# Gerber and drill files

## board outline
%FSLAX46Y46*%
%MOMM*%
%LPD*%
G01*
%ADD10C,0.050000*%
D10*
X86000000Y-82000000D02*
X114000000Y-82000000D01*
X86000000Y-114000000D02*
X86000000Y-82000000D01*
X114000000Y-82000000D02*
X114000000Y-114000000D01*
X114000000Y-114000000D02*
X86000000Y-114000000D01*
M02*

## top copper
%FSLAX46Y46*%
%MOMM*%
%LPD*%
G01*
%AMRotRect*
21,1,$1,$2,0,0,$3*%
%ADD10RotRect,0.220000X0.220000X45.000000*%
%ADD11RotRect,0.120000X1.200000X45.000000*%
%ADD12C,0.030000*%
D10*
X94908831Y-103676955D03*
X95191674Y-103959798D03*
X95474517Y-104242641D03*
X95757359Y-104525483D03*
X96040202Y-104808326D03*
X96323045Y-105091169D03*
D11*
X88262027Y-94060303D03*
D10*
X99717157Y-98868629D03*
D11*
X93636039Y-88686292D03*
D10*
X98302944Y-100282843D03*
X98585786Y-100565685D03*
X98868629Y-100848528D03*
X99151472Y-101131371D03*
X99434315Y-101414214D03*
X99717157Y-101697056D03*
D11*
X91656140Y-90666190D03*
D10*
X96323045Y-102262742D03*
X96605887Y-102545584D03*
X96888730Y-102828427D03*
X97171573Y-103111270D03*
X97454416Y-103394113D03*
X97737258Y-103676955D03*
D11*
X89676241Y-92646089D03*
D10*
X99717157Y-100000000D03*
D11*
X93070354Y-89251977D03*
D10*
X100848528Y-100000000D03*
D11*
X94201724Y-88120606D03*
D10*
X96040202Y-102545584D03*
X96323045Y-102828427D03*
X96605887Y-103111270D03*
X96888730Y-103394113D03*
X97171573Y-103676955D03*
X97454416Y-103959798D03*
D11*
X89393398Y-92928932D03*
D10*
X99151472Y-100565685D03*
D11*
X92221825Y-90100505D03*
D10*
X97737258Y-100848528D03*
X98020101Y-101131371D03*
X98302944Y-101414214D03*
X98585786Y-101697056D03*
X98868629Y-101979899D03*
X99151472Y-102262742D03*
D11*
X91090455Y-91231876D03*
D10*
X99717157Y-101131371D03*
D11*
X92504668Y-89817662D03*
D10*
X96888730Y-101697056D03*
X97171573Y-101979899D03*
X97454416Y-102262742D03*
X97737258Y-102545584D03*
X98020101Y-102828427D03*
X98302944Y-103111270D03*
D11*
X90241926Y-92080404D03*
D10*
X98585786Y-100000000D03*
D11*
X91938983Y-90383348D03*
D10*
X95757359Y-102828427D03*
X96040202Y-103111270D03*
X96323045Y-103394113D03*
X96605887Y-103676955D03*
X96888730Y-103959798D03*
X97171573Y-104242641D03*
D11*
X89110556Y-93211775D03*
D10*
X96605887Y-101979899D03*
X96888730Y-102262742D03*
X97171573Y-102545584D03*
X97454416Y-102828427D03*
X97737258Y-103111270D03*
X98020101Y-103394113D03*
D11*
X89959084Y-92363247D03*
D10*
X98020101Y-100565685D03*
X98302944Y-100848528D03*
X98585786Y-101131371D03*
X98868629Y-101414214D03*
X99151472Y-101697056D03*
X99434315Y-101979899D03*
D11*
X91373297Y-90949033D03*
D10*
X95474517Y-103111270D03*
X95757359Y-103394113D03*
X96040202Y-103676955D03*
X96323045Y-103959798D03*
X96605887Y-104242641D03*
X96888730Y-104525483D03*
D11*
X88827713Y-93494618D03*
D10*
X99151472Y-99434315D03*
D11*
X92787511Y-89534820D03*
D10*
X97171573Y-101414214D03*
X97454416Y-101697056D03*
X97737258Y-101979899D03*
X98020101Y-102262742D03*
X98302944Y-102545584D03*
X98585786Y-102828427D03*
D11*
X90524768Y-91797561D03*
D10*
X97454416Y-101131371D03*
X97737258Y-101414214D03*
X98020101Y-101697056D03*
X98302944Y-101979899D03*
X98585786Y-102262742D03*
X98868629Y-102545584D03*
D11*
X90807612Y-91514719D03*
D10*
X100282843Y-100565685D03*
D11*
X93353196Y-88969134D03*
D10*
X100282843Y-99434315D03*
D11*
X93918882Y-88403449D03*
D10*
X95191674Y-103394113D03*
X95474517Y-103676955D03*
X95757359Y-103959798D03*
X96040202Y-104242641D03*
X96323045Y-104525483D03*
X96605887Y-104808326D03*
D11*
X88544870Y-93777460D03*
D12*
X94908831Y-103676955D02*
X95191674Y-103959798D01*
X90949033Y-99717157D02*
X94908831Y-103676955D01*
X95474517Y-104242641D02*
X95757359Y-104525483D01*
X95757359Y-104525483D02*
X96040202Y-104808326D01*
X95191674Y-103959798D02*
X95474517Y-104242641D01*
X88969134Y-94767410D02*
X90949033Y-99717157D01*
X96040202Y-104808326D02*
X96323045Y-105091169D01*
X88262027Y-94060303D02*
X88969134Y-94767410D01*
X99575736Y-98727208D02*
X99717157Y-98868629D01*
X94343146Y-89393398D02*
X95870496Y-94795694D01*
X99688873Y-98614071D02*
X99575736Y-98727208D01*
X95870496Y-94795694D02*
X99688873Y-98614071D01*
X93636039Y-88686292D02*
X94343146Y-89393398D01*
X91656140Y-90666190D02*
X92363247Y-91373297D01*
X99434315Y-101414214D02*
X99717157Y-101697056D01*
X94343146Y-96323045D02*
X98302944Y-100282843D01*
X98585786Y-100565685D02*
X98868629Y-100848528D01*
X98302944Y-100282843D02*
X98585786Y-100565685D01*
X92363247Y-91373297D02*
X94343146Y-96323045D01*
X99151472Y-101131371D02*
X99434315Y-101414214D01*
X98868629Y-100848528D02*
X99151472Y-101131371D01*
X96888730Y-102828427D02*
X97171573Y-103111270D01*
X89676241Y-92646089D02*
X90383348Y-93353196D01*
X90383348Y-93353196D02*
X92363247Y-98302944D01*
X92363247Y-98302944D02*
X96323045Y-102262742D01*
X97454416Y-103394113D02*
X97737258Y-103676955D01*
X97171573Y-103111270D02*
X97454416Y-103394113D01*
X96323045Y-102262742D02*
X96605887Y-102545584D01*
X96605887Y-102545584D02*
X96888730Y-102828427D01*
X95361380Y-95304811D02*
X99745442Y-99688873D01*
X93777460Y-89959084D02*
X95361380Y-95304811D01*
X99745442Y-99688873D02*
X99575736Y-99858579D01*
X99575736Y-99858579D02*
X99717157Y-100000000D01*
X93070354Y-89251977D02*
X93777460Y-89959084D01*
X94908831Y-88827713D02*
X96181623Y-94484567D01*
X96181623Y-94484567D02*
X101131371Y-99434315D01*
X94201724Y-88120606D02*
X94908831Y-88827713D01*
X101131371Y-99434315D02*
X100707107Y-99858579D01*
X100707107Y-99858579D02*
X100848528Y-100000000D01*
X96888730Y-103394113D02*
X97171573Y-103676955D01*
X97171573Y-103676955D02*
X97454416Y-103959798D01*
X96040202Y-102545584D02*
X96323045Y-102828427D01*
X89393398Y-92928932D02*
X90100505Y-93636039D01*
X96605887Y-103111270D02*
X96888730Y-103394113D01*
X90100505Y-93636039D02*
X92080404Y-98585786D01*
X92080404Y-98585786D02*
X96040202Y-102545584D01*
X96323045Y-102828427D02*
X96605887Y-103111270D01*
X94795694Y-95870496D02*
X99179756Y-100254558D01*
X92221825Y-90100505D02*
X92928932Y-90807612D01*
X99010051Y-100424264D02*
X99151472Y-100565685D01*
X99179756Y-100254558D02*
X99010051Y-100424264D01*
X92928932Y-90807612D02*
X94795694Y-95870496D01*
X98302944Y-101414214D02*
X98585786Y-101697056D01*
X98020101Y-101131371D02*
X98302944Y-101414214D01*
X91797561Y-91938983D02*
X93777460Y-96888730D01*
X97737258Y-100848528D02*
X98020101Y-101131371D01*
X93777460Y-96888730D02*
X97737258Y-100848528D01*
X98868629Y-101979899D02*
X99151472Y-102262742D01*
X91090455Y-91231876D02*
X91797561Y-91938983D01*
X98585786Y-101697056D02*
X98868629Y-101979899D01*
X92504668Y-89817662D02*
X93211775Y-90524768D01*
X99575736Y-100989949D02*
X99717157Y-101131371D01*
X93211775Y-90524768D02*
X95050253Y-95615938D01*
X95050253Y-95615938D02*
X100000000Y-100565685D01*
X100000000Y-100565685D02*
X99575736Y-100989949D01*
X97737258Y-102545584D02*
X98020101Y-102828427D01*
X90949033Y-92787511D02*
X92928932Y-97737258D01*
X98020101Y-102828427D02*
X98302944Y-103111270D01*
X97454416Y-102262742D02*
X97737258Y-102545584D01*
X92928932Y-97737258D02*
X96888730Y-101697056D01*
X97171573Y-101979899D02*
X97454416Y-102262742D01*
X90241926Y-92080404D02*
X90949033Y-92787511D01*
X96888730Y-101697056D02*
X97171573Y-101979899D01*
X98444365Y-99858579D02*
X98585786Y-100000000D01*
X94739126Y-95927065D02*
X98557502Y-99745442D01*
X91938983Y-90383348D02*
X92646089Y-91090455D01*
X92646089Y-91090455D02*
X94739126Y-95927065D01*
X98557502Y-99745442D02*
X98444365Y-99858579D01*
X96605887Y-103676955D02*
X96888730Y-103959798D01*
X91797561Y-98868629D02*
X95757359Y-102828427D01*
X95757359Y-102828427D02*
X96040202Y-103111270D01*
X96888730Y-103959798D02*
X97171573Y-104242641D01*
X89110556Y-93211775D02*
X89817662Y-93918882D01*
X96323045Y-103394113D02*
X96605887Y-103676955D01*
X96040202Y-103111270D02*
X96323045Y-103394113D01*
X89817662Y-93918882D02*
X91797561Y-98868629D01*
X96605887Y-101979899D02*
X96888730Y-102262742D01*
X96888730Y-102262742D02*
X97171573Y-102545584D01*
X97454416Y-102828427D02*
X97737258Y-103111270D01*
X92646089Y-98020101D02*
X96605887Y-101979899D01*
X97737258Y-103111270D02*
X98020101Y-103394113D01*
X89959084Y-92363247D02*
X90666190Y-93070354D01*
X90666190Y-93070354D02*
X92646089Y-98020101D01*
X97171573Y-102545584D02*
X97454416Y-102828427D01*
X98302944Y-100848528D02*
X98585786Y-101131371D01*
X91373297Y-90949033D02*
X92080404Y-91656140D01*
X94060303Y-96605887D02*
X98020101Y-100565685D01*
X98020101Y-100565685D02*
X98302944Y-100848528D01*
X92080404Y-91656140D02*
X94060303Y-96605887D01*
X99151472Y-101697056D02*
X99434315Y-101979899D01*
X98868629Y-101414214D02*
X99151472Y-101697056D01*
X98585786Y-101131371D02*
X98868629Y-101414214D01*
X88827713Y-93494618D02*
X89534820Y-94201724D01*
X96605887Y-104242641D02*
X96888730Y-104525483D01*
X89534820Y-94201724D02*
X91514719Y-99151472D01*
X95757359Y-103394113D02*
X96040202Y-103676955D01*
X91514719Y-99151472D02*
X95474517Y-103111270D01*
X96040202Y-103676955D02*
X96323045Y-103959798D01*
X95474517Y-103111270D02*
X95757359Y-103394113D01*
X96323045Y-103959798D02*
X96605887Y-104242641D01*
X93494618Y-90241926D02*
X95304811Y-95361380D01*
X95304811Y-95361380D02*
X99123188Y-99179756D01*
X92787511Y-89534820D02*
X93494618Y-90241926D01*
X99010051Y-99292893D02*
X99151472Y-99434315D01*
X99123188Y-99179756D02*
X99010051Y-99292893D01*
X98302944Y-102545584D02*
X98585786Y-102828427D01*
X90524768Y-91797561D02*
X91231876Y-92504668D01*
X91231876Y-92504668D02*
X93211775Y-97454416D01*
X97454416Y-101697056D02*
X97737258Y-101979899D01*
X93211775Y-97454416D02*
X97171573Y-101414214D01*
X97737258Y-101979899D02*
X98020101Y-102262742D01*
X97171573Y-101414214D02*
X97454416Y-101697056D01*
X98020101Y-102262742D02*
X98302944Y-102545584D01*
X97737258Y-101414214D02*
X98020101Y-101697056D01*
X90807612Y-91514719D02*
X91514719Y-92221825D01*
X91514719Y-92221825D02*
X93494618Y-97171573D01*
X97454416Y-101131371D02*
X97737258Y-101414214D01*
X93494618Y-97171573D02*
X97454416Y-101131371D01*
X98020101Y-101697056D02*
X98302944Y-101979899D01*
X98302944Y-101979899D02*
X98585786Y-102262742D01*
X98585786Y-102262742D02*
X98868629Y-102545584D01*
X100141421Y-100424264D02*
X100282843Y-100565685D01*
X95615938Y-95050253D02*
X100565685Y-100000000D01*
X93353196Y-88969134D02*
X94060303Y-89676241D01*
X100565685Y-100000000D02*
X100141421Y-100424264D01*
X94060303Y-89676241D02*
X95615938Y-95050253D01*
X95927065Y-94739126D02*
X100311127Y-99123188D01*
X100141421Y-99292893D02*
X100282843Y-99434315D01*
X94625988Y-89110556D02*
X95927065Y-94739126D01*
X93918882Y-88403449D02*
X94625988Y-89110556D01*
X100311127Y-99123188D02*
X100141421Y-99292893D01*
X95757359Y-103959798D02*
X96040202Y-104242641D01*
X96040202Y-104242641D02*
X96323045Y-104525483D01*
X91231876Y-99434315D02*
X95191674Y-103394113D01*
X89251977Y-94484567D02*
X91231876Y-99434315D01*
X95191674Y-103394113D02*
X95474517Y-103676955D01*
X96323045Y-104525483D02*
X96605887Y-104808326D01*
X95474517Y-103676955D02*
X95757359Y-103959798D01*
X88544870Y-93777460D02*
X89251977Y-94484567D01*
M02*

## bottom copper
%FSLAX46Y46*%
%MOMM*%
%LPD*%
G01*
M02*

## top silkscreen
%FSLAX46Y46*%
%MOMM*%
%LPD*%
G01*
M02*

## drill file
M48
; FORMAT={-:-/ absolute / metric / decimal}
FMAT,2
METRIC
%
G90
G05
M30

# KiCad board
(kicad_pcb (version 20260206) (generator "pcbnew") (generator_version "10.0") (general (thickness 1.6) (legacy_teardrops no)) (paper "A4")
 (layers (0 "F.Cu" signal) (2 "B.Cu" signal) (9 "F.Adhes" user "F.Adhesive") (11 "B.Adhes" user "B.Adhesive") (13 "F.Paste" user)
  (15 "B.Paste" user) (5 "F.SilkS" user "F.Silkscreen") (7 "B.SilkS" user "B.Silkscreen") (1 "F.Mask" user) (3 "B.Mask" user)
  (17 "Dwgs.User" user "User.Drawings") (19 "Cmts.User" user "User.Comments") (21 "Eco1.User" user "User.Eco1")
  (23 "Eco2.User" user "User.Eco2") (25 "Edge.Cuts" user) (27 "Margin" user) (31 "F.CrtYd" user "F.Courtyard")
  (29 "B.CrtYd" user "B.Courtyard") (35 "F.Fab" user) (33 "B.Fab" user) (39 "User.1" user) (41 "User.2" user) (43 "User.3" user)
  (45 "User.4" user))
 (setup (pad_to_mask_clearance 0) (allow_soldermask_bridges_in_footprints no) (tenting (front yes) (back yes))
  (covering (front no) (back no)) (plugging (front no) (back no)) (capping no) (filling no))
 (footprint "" (layer "F.Cu") (at 0 0)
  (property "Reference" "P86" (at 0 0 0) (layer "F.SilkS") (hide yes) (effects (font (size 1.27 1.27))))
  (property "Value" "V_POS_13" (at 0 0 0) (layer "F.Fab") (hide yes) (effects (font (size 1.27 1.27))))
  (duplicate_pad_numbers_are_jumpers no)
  (pad "1" connect rect (at 94.908831 103.676955 45) (size 0.22 0.22) (layers "F.Cu") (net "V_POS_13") (thermal_bridge_angle 45))
  (pad "1" connect rect (at 95.191674 103.959798 45) (size 0.22 0.22) (layers "F.Cu") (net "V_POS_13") (thermal_bridge_angle 45))
  (pad "1" connect rect (at 95.474517 104.242641 45) (size 0.22 0.22) (layers "F.Cu") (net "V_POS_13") (thermal_bridge_angle 45))
  (pad "1" connect rect (at 95.757359 104.525483 45) (size 0.22 0.22) (layers "F.Cu") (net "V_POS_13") (thermal_bridge_angle 45))
  (pad "1" connect rect (at 96.040202 104.808326 45) (size 0.22 0.22) (layers "F.Cu") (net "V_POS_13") (thermal_bridge_angle 45))
  (pad "1" connect rect (at 96.323045 105.091169 45) (size 0.22 0.22) (layers "F.Cu") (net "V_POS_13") (thermal_bridge_angle 45))
  (pad "2" connect rect (at 88.262027 94.060303 45) (size 0.12 1.2) (layers "F.Cu") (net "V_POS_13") (thermal_bridge_angle 45)))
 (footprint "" (layer "F.Cu") (at 0 0)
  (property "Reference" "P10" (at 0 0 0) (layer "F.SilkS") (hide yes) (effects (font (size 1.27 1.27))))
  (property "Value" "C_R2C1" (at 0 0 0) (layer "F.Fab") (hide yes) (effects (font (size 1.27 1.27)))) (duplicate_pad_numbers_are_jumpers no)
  (pad "1" connect rect (at 99.717157 98.868629 45) (size 0.22 0.22) (layers "F.Cu") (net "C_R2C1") (thermal_bridge_angle 45))
  (pad "2" connect rect (at 93.636039 88.686292 45) (size 0.12 1.2) (layers "F.Cu") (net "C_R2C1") (thermal_bridge_angle 45)))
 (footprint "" (layer "F.Cu") (at 0 0)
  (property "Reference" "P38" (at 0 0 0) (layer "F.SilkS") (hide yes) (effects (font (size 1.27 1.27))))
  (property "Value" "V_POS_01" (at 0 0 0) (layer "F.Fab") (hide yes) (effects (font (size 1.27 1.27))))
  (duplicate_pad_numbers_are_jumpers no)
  (pad "1" connect rect (at 98.302944 100.282843 45) (size 0.22 0.22) (layers "F.Cu") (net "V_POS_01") (thermal_bridge_angle 45))
  (pad "1" connect rect (at 98.585786 100.565685 45) (size 0.22 0.22) (layers "F.Cu") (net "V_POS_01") (thermal_bridge_angle 45))
  (pad "1" connect rect (at 98.868629 100.848528 45) (size 0.22 0.22) (layers "F.Cu") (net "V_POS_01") (thermal_bridge_angle 45))
  (pad "1" connect rect (at 99.151472 101.131371 45) (size 0.22 0.22) (layers "F.Cu") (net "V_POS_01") (thermal_bridge_angle 45))
  (pad "1" connect rect (at 99.434315 101.414214 45) (size 0.22 0.22) (layers "F.Cu") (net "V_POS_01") (thermal_bridge_angle 45))
  (pad "1" connect rect (at 99.717157 101.697056 45) (size 0.22 0.22) (layers "F.Cu") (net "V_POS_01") (thermal_bridge_angle 45))
  (pad "2" connect rect (at 91.65614 90.66619 45) (size 0.12 1.2) (layers "F.Cu") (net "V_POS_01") (thermal_bridge_angle 45)))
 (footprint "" (layer "F.Cu") (at 0 0)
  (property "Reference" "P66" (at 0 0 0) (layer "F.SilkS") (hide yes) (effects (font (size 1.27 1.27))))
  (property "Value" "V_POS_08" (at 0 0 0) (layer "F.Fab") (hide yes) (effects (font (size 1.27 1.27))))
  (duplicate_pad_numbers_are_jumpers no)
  (pad "1" connect rect (at 96.323045 102.262742 45) (size 0.22 0.22) (layers "F.Cu") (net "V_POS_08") (thermal_bridge_angle 45))
  (pad "1" connect rect (at 96.605887 102.545584 45) (size 0.22 0.22) (layers "F.Cu") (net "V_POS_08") (thermal_bridge_angle 45))
  (pad "1" connect rect (at 96.88873 102.828427 45) (size 0.22 0.22) (layers "F.Cu") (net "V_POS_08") (thermal_bridge_angle 45))
  (pad "1" connect rect (at 97.171573 103.11127 45) (size 0.22 0.22) (layers "F.Cu") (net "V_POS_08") (thermal_bridge_angle 45))
  (pad "1" connect rect (at 97.454416 103.394113 45) (size 0.22 0.22) (layers "F.Cu") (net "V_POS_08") (thermal_bridge_angle 45))
  (pad "1" connect rect (at 97.737258 103.676955 45) (size 0.22 0.22) (layers "F.Cu") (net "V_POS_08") (thermal_bridge_angle 45))
  (pad "2" connect rect (at 89.676241 92.646089 45) (size 0.12 1.2) (layers "F.Cu") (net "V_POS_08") (thermal_bridge_angle 45)))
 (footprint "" (layer "F.Cu") (at 0 0)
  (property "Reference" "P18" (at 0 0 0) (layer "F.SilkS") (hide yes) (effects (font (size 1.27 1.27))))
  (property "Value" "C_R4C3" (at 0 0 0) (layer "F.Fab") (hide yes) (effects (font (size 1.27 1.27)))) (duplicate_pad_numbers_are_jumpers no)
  (pad "1" connect rect (at 99.717157 100 45) (size 0.22 0.22) (layers "F.Cu") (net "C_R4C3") (thermal_bridge_angle 45))
  (pad "2" connect rect (at 93.070354 89.251977 45) (size 0.12 1.2) (layers "F.Cu") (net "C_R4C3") (thermal_bridge_angle 45)))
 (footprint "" (layer "F.Cu") (at 0 0)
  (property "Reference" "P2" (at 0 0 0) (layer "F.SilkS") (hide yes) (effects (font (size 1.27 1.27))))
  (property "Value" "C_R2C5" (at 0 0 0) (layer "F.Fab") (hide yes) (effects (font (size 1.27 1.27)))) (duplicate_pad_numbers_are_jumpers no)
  (pad "1" connect rect (at 100.848528 100 45) (size 0.22 0.22) (layers "F.Cu") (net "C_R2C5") (thermal_bridge_angle 45))
  (pad "2" connect rect (at 94.201724 88.120606 45) (size 0.12 1.2) (layers "F.Cu") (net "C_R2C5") (thermal_bridge_angle 45)))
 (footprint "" (layer "F.Cu") (at 0 0)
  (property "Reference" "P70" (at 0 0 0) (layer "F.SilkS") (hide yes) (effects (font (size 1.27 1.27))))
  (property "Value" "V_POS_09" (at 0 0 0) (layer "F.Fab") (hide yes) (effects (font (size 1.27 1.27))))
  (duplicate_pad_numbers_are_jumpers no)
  (pad "1" connect rect (at 96.040202 102.545584 45) (size 0.22 0.22) (layers "F.Cu") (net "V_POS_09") (thermal_bridge_angle 45))
  (pad "1" connect rect (at 96.323045 102.828427 45) (size 0.22 0.22) (layers "F.Cu") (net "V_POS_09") (thermal_bridge_angle 45))
  (pad "1" connect rect (at 96.605887 103.11127 45) (size 0.22 0.22) (layers "F.Cu") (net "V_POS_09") (thermal_bridge_angle 45))
  (pad "1" connect rect (at 96.88873 103.394113 45) (size 0.22 0.22) (layers "F.Cu") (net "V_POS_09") (thermal_bridge_angle 45))
  (pad "1" connect rect (at 97.171573 103.676955 45) (size 0.22 0.22) (layers "F.Cu") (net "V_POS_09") (thermal_bridge_angle 45))
  (pad "1" connect rect (at 97.454416 103.959798 45) (size 0.22 0.22) (layers "F.Cu") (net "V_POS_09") (thermal_bridge_angle 45))
  (pad "2" connect rect (at 89.393398 92.928932 45) (size 0.12 1.2) (layers "F.Cu") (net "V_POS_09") (thermal_bridge_angle 45)))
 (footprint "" (layer "F.Cu") (at 0 0)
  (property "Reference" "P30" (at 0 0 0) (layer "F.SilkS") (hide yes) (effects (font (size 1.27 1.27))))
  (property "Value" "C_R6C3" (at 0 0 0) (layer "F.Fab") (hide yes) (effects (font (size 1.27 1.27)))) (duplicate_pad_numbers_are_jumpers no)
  (pad "1" connect rect (at 99.151472 100.565685 45) (size 0.22 0.22) (layers "F.Cu") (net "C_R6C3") (thermal_bridge_angle 45))
  (pad "2" connect rect (at 92.221825 90.100505 45) (size 0.12 1.2) (layers "F.Cu") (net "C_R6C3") (thermal_bridge_angle 45)))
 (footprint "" (layer "F.Cu") (at 0 0)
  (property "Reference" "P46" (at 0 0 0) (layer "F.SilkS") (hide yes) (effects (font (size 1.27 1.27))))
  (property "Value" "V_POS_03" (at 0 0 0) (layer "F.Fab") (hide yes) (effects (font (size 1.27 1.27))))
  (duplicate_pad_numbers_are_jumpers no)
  (pad "1" connect rect (at 97.737258 100.848528 45) (size 0.22 0.22) (layers "F.Cu") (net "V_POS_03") (thermal_bridge_angle 45))
  (pad "1" connect rect (at 98.020101 101.131371 45) (size 0.22 0.22) (layers "F.Cu") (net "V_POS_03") (thermal_bridge_angle 45))
  (pad "1" connect rect (at 98.302944 101.414214 45) (size 0.22 0.22) (layers "F.Cu") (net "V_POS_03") (thermal_bridge_angle 45))
  (pad "1" connect rect (at 98.585786 101.697056 45) (size 0.22 0.22) (layers "F.Cu") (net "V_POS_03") (thermal_bridge_angle 45))
  (pad "1" connect rect (at 98.868629 101.979899 45) (size 0.22 0.22) (layers "F.Cu") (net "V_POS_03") (thermal_bridge_angle 45))
  (pad "1" connect rect (at 99.151472 102.262742 45) (size 0.22 0.22) (layers "F.Cu") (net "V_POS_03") (thermal_bridge_angle 45))
  (pad "2" connect rect (at 91.090455 91.231876 45) (size 0.12 1.2) (layers "F.Cu") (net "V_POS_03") (thermal_bridge_angle 45)))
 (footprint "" (layer "F.Cu") (at 0 0)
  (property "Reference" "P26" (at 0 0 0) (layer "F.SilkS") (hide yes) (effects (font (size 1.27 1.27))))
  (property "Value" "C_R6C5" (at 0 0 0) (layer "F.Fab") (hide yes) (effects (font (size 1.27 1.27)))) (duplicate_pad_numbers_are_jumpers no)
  (pad "1" connect rect (at 99.717157 101.131371 45) (size 0.22 0.22) (layers "F.Cu") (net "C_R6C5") (thermal_bridge_angle 45))
  (pad "2" connect rect (at 92.504668 89.817662 45) (size 0.12 1.2) (layers "F.Cu") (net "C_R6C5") (thermal_bridge_angle 45)))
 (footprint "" (layer "F.Cu") (at 0 0)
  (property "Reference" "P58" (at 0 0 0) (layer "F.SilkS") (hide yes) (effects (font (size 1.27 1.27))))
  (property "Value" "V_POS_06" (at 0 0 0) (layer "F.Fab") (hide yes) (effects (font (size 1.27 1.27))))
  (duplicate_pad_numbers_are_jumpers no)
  (pad "1" connect rect (at 96.88873 101.697056 45) (size 0.22 0.22) (layers "F.Cu") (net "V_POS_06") (thermal_bridge_angle 45))
  (pad "1" connect rect (at 97.171573 101.979899 45) (size 0.22 0.22) (layers "F.Cu") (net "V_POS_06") (thermal_bridge_angle 45))
  (pad "1" connect rect (at 97.454416 102.262742 45) (size 0.22 0.22) (layers "F.Cu") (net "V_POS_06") (thermal_bridge_angle 45))
  (pad "1" connect rect (at 97.737258 102.545584 45) (size 0.22 0.22) (layers "F.Cu") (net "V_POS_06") (thermal_bridge_angle 45))
  (pad "1" connect rect (at 98.020101 102.828427 45) (size 0.22 0.22) (layers "F.Cu") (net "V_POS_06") (thermal_bridge_angle 45))
  (pad "1" connect rect (at 98.302944 103.11127 45) (size 0.22 0.22) (layers "F.Cu") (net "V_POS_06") (thermal_bridge_angle 45))
  (pad "2" connect rect (at 90.241926 92.080404 45) (size 0.12 1.2) (layers "F.Cu") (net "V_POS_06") (thermal_bridge_angle 45)))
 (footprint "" (layer "F.Cu") (at 0 0)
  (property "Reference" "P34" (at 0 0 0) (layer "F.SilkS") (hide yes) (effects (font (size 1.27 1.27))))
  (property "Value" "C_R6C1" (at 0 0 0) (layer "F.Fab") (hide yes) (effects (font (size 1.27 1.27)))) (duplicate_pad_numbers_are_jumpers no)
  (pad "1" connect rect (at 98.585786 100 45) (size 0.22 0.22) (layers "F.Cu") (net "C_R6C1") (thermal_bridge_angle 45))
  (pad "2" connect rect (at 91.938983 90.383348 45) (size 0.12 1.2) (layers "F.Cu") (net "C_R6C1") (thermal_bridge_angle 45)))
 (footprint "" (layer "F.Cu") (at 0 0)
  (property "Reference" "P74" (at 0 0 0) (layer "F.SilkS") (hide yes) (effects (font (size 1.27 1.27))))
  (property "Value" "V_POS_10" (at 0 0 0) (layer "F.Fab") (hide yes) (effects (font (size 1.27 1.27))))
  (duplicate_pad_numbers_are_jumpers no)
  (pad "1" connect rect (at 95.757359 102.828427 45) (size 0.22 0.22) (layers "F.Cu") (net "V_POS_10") (thermal_bridge_angle 45))
  (pad "1" connect rect (at 96.040202 103.11127 45) (size 0.22 0.22) (layers "F.Cu") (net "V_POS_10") (thermal_bridge_angle 45))
  (pad "1" connect rect (at 96.323045 103.394113 45) (size 0.22 0.22) (layers "F.Cu") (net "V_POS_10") (thermal_bridge_angle 45))
  (pad "1" connect rect (at 96.605887 103.676955 45) (size 0.22 0.22) (layers "F.Cu") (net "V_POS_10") (thermal_bridge_angle 45))
  (pad "1" connect rect (at 96.88873 103.959798 45) (size 0.22 0.22) (layers "F.Cu") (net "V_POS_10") (thermal_bridge_angle 45))
  (pad "1" connect rect (at 97.171573 104.242641 45) (size 0.22 0.22) (layers "F.Cu") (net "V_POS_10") (thermal_bridge_angle 45))
  (pad "2" connect rect (at 89.110556 93.211775 45) (size 0.12 1.2) (layers "F.Cu") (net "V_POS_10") (thermal_bridge_angle 45)))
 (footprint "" (layer "F.Cu") (at 0 0)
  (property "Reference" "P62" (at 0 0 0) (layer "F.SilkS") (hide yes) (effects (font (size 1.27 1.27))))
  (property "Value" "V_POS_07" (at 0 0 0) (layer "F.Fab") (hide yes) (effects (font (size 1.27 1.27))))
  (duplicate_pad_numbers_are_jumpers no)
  (pad "1" connect rect (at 96.605887 101.979899 45) (size 0.22 0.22) (layers "F.Cu") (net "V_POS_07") (thermal_bridge_angle 45))
  (pad "1" connect rect (at 96.88873 102.262742 45) (size 0.22 0.22) (layers "F.Cu") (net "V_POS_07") (thermal_bridge_angle 45))
  (pad "1" connect rect (at 97.171573 102.545584 45) (size 0.22 0.22) (layers "F.Cu") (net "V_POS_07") (thermal_bridge_angle 45))
  (pad "1" connect rect (at 97.454416 102.828427 45) (size 0.22 0.22) (layers "F.Cu") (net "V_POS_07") (thermal_bridge_angle 45))
  (pad "1" connect rect (at 97.737258 103.11127 45) (size 0.22 0.22) (layers "F.Cu") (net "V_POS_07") (thermal_bridge_angle 45))
  (pad "1" connect rect (at 98.020101 103.394113 45) (size 0.22 0.22) (layers "F.Cu") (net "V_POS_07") (thermal_bridge_angle 45))
  (pad "2" connect rect (at 89.959084 92.363247 45) (size 0.12 1.2) (layers "F.Cu") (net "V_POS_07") (thermal_bridge_angle 45)))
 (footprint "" (layer "F.Cu") (at 0 0)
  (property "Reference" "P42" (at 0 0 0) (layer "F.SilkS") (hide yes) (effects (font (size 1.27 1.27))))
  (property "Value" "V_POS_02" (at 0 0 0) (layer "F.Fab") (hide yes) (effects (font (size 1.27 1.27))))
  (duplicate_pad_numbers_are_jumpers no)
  (pad "1" connect rect (at 98.020101 100.565685 45) (size 0.22 0.22) (layers "F.Cu") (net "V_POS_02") (thermal_bridge_angle 45))
  (pad "1" connect rect (at 98.302944 100.848528 45) (size 0.22 0.22) (layers "F.Cu") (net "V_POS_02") (thermal_bridge_angle 45))
  (pad "1" connect rect (at 98.585786 101.131371 45) (size 0.22 0.22) (layers "F.Cu") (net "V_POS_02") (thermal_bridge_angle 45))
  (pad "1" connect rect (at 98.868629 101.414214 45) (size 0.22 0.22) (layers "F.Cu") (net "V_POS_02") (thermal_bridge_angle 45))
  (pad "1" connect rect (at 99.151472 101.697056 45) (size 0.22 0.22) (layers "F.Cu") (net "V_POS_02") (thermal_bridge_angle 45))
  (pad "1" connect rect (at 99.434315 101.979899 45) (size 0.22 0.22) (layers "F.Cu") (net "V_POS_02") (thermal_bridge_angle 45))
  (pad "2" connect rect (at 91.373297 90.949033 45) (size 0.12 1.2) (layers "F.Cu") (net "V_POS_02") (thermal_bridge_angle 45)))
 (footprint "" (layer "F.Cu") (at 0 0)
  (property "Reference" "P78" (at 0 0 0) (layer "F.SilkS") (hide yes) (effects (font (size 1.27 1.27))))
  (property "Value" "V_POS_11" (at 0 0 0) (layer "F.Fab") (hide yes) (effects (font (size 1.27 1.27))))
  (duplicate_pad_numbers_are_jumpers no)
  (pad "1" connect rect (at 95.474517 103.11127 45) (size 0.22 0.22) (layers "F.Cu") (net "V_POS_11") (thermal_bridge_angle 45))
  (pad "1" connect rect (at 95.757359 103.394113 45) (size 0.22 0.22) (layers "F.Cu") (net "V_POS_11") (thermal_bridge_angle 45))
  (pad "1" connect rect (at 96.040202 103.676955 45) (size 0.22 0.22) (layers "F.Cu") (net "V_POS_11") (thermal_bridge_angle 45))
  (pad "1" connect rect (at 96.323045 103.959798 45) (size 0.22 0.22) (layers "F.Cu") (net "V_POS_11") (thermal_bridge_angle 45))
  (pad "1" connect rect (at 96.605887 104.242641 45) (size 0.22 0.22) (layers "F.Cu") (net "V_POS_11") (thermal_bridge_angle 45))
  (pad "1" connect rect (at 96.88873 104.525483 45) (size 0.22 0.22) (layers "F.Cu") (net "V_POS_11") (thermal_bridge_angle 45))
  (pad "2" connect rect (at 88.827713 93.494618 45) (size 0.12 1.2) (layers "F.Cu") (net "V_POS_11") (thermal_bridge_angle 45)))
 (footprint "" (layer "F.Cu") (at 0 0)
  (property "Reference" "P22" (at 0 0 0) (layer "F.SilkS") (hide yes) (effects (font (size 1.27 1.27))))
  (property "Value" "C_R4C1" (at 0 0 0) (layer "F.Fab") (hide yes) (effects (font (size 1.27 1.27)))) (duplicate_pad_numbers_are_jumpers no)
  (pad "1" connect rect (at 99.151472 99.434315 45) (size 0.22 0.22) (layers "F.Cu") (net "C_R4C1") (thermal_bridge_angle 45))
  (pad "2" connect rect (at 92.787511 89.53482 45) (size 0.12 1.2) (layers "F.Cu") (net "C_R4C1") (thermal_bridge_angle 45)))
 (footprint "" (layer "F.Cu") (at 0 0)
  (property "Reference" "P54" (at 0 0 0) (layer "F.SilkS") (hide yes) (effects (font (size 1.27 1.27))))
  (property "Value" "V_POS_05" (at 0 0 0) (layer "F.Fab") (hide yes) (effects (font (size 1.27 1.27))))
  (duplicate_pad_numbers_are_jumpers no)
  (pad "1" connect rect (at 97.171573 101.414214 45) (size 0.22 0.22) (layers "F.Cu") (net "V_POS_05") (thermal_bridge_angle 45))
  (pad "1" connect rect (at 97.454416 101.697056 45) (size 0.22 0.22) (layers "F.Cu") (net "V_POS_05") (thermal_bridge_angle 45))
  (pad "1" connect rect (at 97.737258 101.979899 45) (size 0.22 0.22) (layers "F.Cu") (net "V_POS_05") (thermal_bridge_angle 45))
  (pad "1" connect rect (at 98.020101 102.262742 45) (size 0.22 0.22) (layers "F.Cu") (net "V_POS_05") (thermal_bridge_angle 45))
  (pad "1" connect rect (at 98.302944 102.545584 45) (size 0.22 0.22) (layers "F.Cu") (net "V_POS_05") (thermal_bridge_angle 45))
  (pad "1" connect rect (at 98.585786 102.828427 45) (size 0.22 0.22) (layers "F.Cu") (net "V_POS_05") (thermal_bridge_angle 45))
  (pad "2" connect rect (at 90.524768 91.797561 45) (size 0.12 1.2) (layers "F.Cu") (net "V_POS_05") (thermal_bridge_angle 45)))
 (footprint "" (layer "F.Cu") (at 0 0)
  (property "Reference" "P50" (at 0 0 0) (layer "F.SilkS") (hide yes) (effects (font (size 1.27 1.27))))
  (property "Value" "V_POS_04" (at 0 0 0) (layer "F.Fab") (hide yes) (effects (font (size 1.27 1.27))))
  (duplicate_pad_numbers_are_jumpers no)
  (pad "1" connect rect (at 97.454416 101.131371 45) (size 0.22 0.22) (layers "F.Cu") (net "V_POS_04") (thermal_bridge_angle 45))
  (pad "1" connect rect (at 97.737258 101.414214 45) (size 0.22 0.22) (layers "F.Cu") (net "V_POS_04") (thermal_bridge_angle 45))
  (pad "1" connect rect (at 98.020101 101.697056 45) (size 0.22 0.22) (layers "F.Cu") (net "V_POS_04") (thermal_bridge_angle 45))
  (pad "1" connect rect (at 98.302944 101.979899 45) (size 0.22 0.22) (layers "F.Cu") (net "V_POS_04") (thermal_bridge_angle 45))
  (pad "1" connect rect (at 98.585786 102.262742 45) (size 0.22 0.22) (layers "F.Cu") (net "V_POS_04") (thermal_bridge_angle 45))
  (pad "1" connect rect (at 98.868629 102.545584 45) (size 0.22 0.22) (layers "F.Cu") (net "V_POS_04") (thermal_bridge_angle 45))
  (pad "2" connect rect (at 90.807612 91.514719 45) (size 0.12 1.2) (layers "F.Cu") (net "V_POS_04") (thermal_bridge_angle 45)))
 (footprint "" (layer "F.Cu") (at 0 0)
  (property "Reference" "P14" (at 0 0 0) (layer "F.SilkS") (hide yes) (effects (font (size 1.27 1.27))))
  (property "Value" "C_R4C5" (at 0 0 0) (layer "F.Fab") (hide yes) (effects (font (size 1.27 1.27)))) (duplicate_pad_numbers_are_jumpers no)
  (pad "1" connect rect (at 100.282843 100.565685 45) (size 0.22 0.22) (layers "F.Cu") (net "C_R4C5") (thermal_bridge_angle 45))
  (pad "2" connect rect (at 93.353196 88.969134 45) (size 0.12 1.2) (layers "F.Cu") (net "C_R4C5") (thermal_bridge_angle 45)))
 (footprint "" (layer "F.Cu") (at 0 0)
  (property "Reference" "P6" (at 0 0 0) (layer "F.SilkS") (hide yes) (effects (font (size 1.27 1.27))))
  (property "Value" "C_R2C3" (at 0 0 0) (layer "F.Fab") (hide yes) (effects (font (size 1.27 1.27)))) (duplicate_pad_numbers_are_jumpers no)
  (pad "1" connect rect (at 100.282843 99.434315 45) (size 0.22 0.22) (layers "F.Cu") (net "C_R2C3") (thermal_bridge_angle 45))
  (pad "2" connect rect (at 93.918882 88.403449 45) (size 0.12 1.2) (layers "F.Cu") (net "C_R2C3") (thermal_bridge_angle 45)))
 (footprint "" (layer "F.Cu") (at 0 0)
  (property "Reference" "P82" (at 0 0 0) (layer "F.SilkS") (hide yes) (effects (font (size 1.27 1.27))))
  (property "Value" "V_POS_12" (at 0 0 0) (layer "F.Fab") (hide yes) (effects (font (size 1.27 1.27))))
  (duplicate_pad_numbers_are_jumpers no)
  (pad "1" connect rect (at 95.191674 103.394113 45) (size 0.22 0.22) (layers "F.Cu") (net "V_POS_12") (thermal_bridge_angle 45))
  (pad "1" connect rect (at 95.474517 103.676955 45) (size 0.22 0.22) (layers "F.Cu") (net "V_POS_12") (thermal_bridge_angle 45))
  (pad "1" connect rect (at 95.757359 103.959798 45) (size 0.22 0.22) (layers "F.Cu") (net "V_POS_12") (thermal_bridge_angle 45))
  (pad "1" connect rect (at 96.040202 104.242641 45) (size 0.22 0.22) (layers "F.Cu") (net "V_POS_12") (thermal_bridge_angle 45))
  (pad "1" connect rect (at 96.323045 104.525483 45) (size 0.22 0.22) (layers "F.Cu") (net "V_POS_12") (thermal_bridge_angle 45))
  (pad "1" connect rect (at 96.605887 104.808326 45) (size 0.22 0.22) (layers "F.Cu") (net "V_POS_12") (thermal_bridge_angle 45))
  (pad "2" connect rect (at 88.54487 93.77746 45) (size 0.12 1.2) (layers "F.Cu") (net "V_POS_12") (thermal_bridge_angle 45)))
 (gr_line (start 86 82) (end 114 82) (stroke (width 0.05) (type default)) (layer "Edge.Cuts"))
 (gr_line (start 86 114) (end 86 82) (stroke (width 0.05) (type default)) (layer "Edge.Cuts"))
 (gr_line (start 114 82) (end 114 114) (stroke (width 0.05) (type default)) (layer "Edge.Cuts"))
 (gr_line (start 114 114) (end 86 114) (stroke (width 0.05) (type default)) (layer "Edge.Cuts"))
 (segment (start 94.908831 103.676955) (end 95.191674 103.959798) (width 0.03) (layer "F.Cu") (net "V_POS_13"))
 (segment (start 90.949033 99.717157) (end 94.908831 103.676955) (width 0.03) (layer "F.Cu") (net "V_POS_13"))
 (segment (start 95.474517 104.242641) (end 95.757359 104.525483) (width 0.03) (layer "F.Cu") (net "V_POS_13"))
 (segment (start 95.757359 104.525483) (end 96.040202 104.808326) (width 0.03) (layer "F.Cu") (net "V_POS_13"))
 (segment (start 95.191674 103.959798) (end 95.474517 104.242641) (width 0.03) (layer "F.Cu") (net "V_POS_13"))
 (segment (start 88.969134 94.76741) (end 90.949033 99.717157) (width 0.03) (layer "F.Cu") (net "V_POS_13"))
 (segment (start 96.040202 104.808326) (end 96.323045 105.091169) (width 0.03) (layer "F.Cu") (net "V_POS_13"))
 (segment (start 88.262027 94.060303) (end 88.969134 94.76741) (width 0.03) (layer "F.Cu") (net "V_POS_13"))
 (segment (start 99.575736 98.727208) (end 99.717157 98.868629) (width 0.03) (layer "F.Cu") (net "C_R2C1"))
 (segment (start 94.343146 89.393398) (end 95.870496 94.795694) (width 0.03) (layer "F.Cu") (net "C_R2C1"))
 (segment (start 99.688873 98.614071) (end 99.575736 98.727208) (width 0.03) (layer "F.Cu") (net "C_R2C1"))
 (segment (start 95.870496 94.795694) (end 99.688873 98.614071) (width 0.03) (layer "F.Cu") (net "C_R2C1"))
 (segment (start 93.636039 88.686292) (end 94.343146 89.393398) (width 0.03) (layer "F.Cu") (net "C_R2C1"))
 (segment (start 91.65614 90.66619) (end 92.363247 91.373297) (width 0.03) (layer "F.Cu") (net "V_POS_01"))
 (segment (start 99.434315 101.414214) (end 99.717157 101.697056) (width 0.03) (layer "F.Cu") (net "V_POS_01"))
 (segment (start 94.343146 96.323045) (end 98.302944 100.282843) (width 0.03) (layer "F.Cu") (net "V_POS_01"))
 (segment (start 98.585786 100.565685) (end 98.868629 100.848528) (width 0.03) (layer "F.Cu") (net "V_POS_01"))
 (segment (start 98.302944 100.282843) (end 98.585786 100.565685) (width 0.03) (layer "F.Cu") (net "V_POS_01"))
 (segment (start 92.363247 91.373297) (end 94.343146 96.323045) (width 0.03) (layer "F.Cu") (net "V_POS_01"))
 (segment (start 99.151472 101.131371) (end 99.434315 101.414214) (width 0.03) (layer "F.Cu") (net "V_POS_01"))
 (segment (start 98.868629 100.848528) (end 99.151472 101.131371) (width 0.03) (layer "F.Cu") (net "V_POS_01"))
 (segment (start 96.88873 102.828427) (end 97.171573 103.11127) (width 0.03) (layer "F.Cu") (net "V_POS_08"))
 (segment (start 89.676241 92.646089) (end 90.383348 93.353196) (width 0.03) (layer "F.Cu") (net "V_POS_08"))
 (segment (start 90.383348 93.353196) (end 92.363247 98.302944) (width 0.03) (layer "F.Cu") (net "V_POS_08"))
 (segment (start 92.363247 98.302944) (end 96.323045 102.262742) (width 0.03) (layer "F.Cu") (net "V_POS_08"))
 (segment (start 97.454416 103.394113) (end 97.737258 103.676955) (width 0.03) (layer "F.Cu") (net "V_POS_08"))
 (segment (start 97.171573 103.11127) (end 97.454416 103.394113) (width 0.03) (layer "F.Cu") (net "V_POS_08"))
 (segment (start 96.323045 102.262742) (end 96.605887 102.545584) (width 0.03) (layer "F.Cu") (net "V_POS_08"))
 (segment (start 96.605887 102.545584) (end 96.88873 102.828427) (width 0.03) (layer "F.Cu") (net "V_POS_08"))
 (segment (start 95.36138 95.304811) (end 99.745442 99.688873) (width 0.03) (layer "F.Cu") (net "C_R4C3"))
 (segment (start 93.77746 89.959084) (end 95.36138 95.304811) (width 0.03) (layer "F.Cu") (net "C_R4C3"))
 (segment (start 99.745442 99.688873) (end 99.575736 99.858579) (width 0.03) (layer "F.Cu") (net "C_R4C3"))
 (segment (start 99.575736 99.858579) (end 99.717157 100) (width 0.03) (layer "F.Cu") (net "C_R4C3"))
 (segment (start 93.070354 89.251977) (end 93.77746 89.959084) (width 0.03) (layer "F.Cu") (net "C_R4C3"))
 (segment (start 94.908831 88.827713) (end 96.181623 94.484567) (width 0.03) (layer "F.Cu") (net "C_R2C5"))
 (segment (start 96.181623 94.484567) (end 101.131371 99.434315) (width 0.03) (layer "F.Cu") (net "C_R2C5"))
 (segment (start 94.201724 88.120606) (end 94.908831 88.827713) (width 0.03) (layer "F.Cu") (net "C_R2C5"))
 (segment (start 101.131371 99.434315) (end 100.707107 99.858579) (width 0.03) (layer "F.Cu") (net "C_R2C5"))
 (segment (start 100.707107 99.858579) (end 100.848528 100) (width 0.03) (layer "F.Cu") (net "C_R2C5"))
 (segment (start 96.88873 103.394113) (end 97.171573 103.676955) (width 0.03) (layer "F.Cu") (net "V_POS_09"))
 (segment (start 97.171573 103.676955) (end 97.454416 103.959798) (width 0.03) (layer "F.Cu") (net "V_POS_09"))
 (segment (start 96.040202 102.545584) (end 96.323045 102.828427) (width 0.03) (layer "F.Cu") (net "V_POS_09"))
 (segment (start 89.393398 92.928932) (end 90.100505 93.636039) (width 0.03) (layer "F.Cu") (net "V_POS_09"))
 (segment (start 96.605887 103.11127) (end 96.88873 103.394113) (width 0.03) (layer "F.Cu") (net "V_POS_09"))
 (segment (start 90.100505 93.636039) (end 92.080404 98.585786) (width 0.03) (layer "F.Cu") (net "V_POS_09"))
 (segment (start 92.080404 98.585786) (end 96.040202 102.545584) (width 0.03) (layer "F.Cu") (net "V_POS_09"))
 (segment (start 96.323045 102.828427) (end 96.605887 103.11127) (width 0.03) (layer "F.Cu") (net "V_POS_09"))
 (segment (start 94.795694 95.870496) (end 99.179756 100.254558) (width 0.03) (layer "F.Cu") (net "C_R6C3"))
 (segment (start 92.221825 90.100505) (end 92.928932 90.807612) (width 0.03) (layer "F.Cu") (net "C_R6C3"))
 (segment (start 99.010051 100.424264) (end 99.151472 100.565685) (width 0.03) (layer "F.Cu") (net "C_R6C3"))
 (segment (start 99.179756 100.254558) (end 99.010051 100.424264) (width 0.03) (layer "F.Cu") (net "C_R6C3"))
 (segment (start 92.928932 90.807612) (end 94.795694 95.870496) (width 0.03) (layer "F.Cu") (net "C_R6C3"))
 (segment (start 98.302944 101.414214) (end 98.585786 101.697056) (width 0.03) (layer "F.Cu") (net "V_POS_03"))
 (segment (start 98.020101 101.131371) (end 98.302944 101.414214) (width 0.03) (layer "F.Cu") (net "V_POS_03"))
 (segment (start 91.797561 91.938983) (end 93.77746 96.88873) (width 0.03) (layer "F.Cu") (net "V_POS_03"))
 (segment (start 97.737258 100.848528) (end 98.020101 101.131371) (width 0.03) (layer "F.Cu") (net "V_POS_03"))
 (segment (start 93.77746 96.88873) (end 97.737258 100.848528) (width 0.03) (layer "F.Cu") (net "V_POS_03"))
 (segment (start 98.868629 101.979899) (end 99.151472 102.262742) (width 0.03) (layer "F.Cu") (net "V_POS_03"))
 (segment (start 91.090455 91.231876) (end 91.797561 91.938983) (width 0.03) (layer "F.Cu") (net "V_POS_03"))
 (segment (start 98.585786 101.697056) (end 98.868629 101.979899) (width 0.03) (layer "F.Cu") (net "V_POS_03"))
 (segment (start 92.504668 89.817662) (end 93.211775 90.524768) (width 0.03) (layer "F.Cu") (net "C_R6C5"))
 (segment (start 99.575736 100.989949) (end 99.717157 101.131371) (width 0.03) (layer "F.Cu") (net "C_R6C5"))
 (segment (start 93.211775 90.524768) (end 95.050253 95.615938) (width 0.03) (layer "F.Cu") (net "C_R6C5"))
 (segment (start 95.050253 95.615938) (end 100 100.565685) (width 0.03) (layer "F.Cu") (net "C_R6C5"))
 (segment (start 100 100.565685) (end 99.575736 100.989949) (width 0.03) (layer "F.Cu") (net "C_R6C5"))
 (segment (start 97.737258 102.545584) (end 98.020101 102.828427) (width 0.03) (layer "F.Cu") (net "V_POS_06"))
 (segment (start 90.949033 92.787511) (end 92.928932 97.737258) (width 0.03) (layer "F.Cu") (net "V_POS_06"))
 (segment (start 98.020101 102.828427) (end 98.302944 103.11127) (width 0.03) (layer "F.Cu") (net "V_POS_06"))
 (segment (start 97.454416 102.262742) (end 97.737258 102.545584) (width 0.03) (layer "F.Cu") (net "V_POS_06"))
 (segment (start 92.928932 97.737258) (end 96.88873 101.697056) (width 0.03) (layer "F.Cu") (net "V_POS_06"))
 (segment (start 97.171573 101.979899) (end 97.454416 102.262742) (width 0.03) (layer "F.Cu") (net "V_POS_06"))
 (segment (start 90.241926 92.080404) (end 90.949033 92.787511) (width 0.03) (layer "F.Cu") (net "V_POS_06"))
 (segment (start 96.88873 101.697056) (end 97.171573 101.979899) (width 0.03) (layer "F.Cu") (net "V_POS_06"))
 (segment (start 98.444365 99.858579) (end 98.585786 100) (width 0.03) (layer "F.Cu") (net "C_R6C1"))
 (segment (start 94.739126 95.927065) (end 98.557502 99.745442) (width 0.03) (layer "F.Cu") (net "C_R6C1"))
 (segment (start 91.938983 90.383348) (end 92.646089 91.090455) (width 0.03) (layer "F.Cu") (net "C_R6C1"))
 (segment (start 92.646089 91.090455) (end 94.739126 95.927065) (width 0.03) (layer "F.Cu") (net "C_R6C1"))
 (segment (start 98.557502 99.745442) (end 98.444365 99.858579) (width 0.03) (layer "F.Cu") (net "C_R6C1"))
 (segment (start 96.605887 103.676955) (end 96.88873 103.959798) (width 0.03) (layer "F.Cu") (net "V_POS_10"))
 (segment (start 91.797561 98.868629) (end 95.757359 102.828427) (width 0.03) (layer "F.Cu") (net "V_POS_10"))
 (segment (start 95.757359 102.828427) (end 96.040202 103.11127) (width 0.03) (layer "F.Cu") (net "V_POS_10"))
 (segment (start 96.88873 103.959798) (end 97.171573 104.242641) (width 0.03) (layer "F.Cu") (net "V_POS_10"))
 (segment (start 89.110556 93.211775) (end 89.817662 93.918882) (width 0.03) (layer "F.Cu") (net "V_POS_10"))
 (segment (start 96.323045 103.394113) (end 96.605887 103.676955) (width 0.03) (layer "F.Cu") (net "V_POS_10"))
 (segment (start 96.040202 103.11127) (end 96.323045 103.394113) (width 0.03) (layer "F.Cu") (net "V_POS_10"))
 (segment (start 89.817662 93.918882) (end 91.797561 98.868629) (width 0.03) (layer "F.Cu") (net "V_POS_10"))
 (segment (start 96.605887 101.979899) (end 96.88873 102.262742) (width 0.03) (layer "F.Cu") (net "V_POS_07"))
 (segment (start 96.88873 102.262742) (end 97.171573 102.545584) (width 0.03) (layer "F.Cu") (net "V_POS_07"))
 (segment (start 97.454416 102.828427) (end 97.737258 103.11127) (width 0.03) (layer "F.Cu") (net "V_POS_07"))
 (segment (start 92.646089 98.020101) (end 96.605887 101.979899) (width 0.03) (layer "F.Cu") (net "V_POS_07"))
 (segment (start 97.737258 103.11127) (end 98.020101 103.394113) (width 0.03) (layer "F.Cu") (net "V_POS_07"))
 (segment (start 89.959084 92.363247) (end 90.66619 93.070354) (width 0.03) (layer "F.Cu") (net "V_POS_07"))
 (segment (start 90.66619 93.070354) (end 92.646089 98.020101) (width 0.03) (layer "F.Cu") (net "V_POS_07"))
 (segment (start 97.171573 102.545584) (end 97.454416 102.828427) (width 0.03) (layer "F.Cu") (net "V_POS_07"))
 (segment (start 98.302944 100.848528) (end 98.585786 101.131371) (width 0.03) (layer "F.Cu") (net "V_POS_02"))
 (segment (start 91.373297 90.949033) (end 92.080404 91.65614) (width 0.03) (layer "F.Cu") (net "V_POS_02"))
 (segment (start 94.060303 96.605887) (end 98.020101 100.565685) (width 0.03) (layer "F.Cu") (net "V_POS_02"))
 (segment (start 98.020101 100.565685) (end 98.302944 100.848528) (width 0.03) (layer "F.Cu") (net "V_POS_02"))
 (segment (start 92.080404 91.65614) (end 94.060303 96.605887) (width 0.03) (layer "F.Cu") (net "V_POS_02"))
 (segment (start 99.151472 101.697056) (end 99.434315 101.979899) (width 0.03) (layer "F.Cu") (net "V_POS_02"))
 (segment (start 98.868629 101.414214) (end 99.151472 101.697056) (width 0.03) (layer "F.Cu") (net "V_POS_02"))
 (segment (start 98.585786 101.131371) (end 98.868629 101.414214) (width 0.03) (layer "F.Cu") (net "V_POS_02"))
 (segment (start 88.827713 93.494618) (end 89.53482 94.201724) (width 0.03) (layer "F.Cu") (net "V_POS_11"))
 (segment (start 96.605887 104.242641) (end 96.88873 104.525483) (width 0.03) (layer "F.Cu") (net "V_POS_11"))
 (segment (start 89.53482 94.201724) (end 91.514719 99.151472) (width 0.03) (layer "F.Cu") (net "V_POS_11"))
 (segment (start 95.757359 103.394113) (end 96.040202 103.676955) (width 0.03) (layer "F.Cu") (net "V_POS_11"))
 (segment (start 91.514719 99.151472) (end 95.474517 103.11127) (width 0.03) (layer "F.Cu") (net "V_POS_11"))
 (segment (start 96.040202 103.676955) (end 96.323045 103.959798) (width 0.03) (layer "F.Cu") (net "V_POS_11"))
 (segment (start 95.474517 103.11127) (end 95.757359 103.394113) (width 0.03) (layer "F.Cu") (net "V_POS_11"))
 (segment (start 96.323045 103.959798) (end 96.605887 104.242641) (width 0.03) (layer "F.Cu") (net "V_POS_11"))
 (segment (start 93.494618 90.241926) (end 95.304811 95.36138) (width 0.03) (layer "F.Cu") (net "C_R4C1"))
 (segment (start 95.304811 95.36138) (end 99.123188 99.179756) (width 0.03) (layer "F.Cu") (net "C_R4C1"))
 (segment (start 92.787511 89.53482) (end 93.494618 90.241926) (width 0.03) (layer "F.Cu") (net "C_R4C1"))
 (segment (start 99.010051 99.292893) (end 99.151472 99.434315) (width 0.03) (layer "F.Cu") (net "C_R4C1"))
 (segment (start 99.123188 99.179756) (end 99.010051 99.292893) (width 0.03) (layer "F.Cu") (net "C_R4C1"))
 (segment (start 98.302944 102.545584) (end 98.585786 102.828427) (width 0.03) (layer "F.Cu") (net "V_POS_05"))
 (segment (start 90.524768 91.797561) (end 91.231876 92.504668) (width 0.03) (layer "F.Cu") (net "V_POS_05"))
 (segment (start 91.231876 92.504668) (end 93.211775 97.454416) (width 0.03) (layer "F.Cu") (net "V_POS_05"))
 (segment (start 97.454416 101.697056) (end 97.737258 101.979899) (width 0.03) (layer "F.Cu") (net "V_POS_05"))
 (segment (start 93.211775 97.454416) (end 97.171573 101.414214) (width 0.03) (layer "F.Cu") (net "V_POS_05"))
 (segment (start 97.737258 101.979899) (end 98.020101 102.262742) (width 0.03) (layer "F.Cu") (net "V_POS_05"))
 (segment (start 97.171573 101.414214) (end 97.454416 101.697056) (width 0.03) (layer "F.Cu") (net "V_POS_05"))
 (segment (start 98.020101 102.262742) (end 98.302944 102.545584) (width 0.03) (layer "F.Cu") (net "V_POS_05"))
 (segment (start 97.737258 101.414214) (end 98.020101 101.697056) (width 0.03) (layer "F.Cu") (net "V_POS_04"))
 (segment (start 90.807612 91.514719) (end 91.514719 92.221825) (width 0.03) (layer "F.Cu") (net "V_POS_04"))
 (segment (start 91.514719 92.221825) (end 93.494618 97.171573) (width 0.03) (layer "F.Cu") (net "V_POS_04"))
 (segment (start 97.454416 101.131371) (end 97.737258 101.414214) (width 0.03) (layer "F.Cu") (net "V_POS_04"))
 (segment (start 93.494618 97.171573) (end 97.454416 101.131371) (width 0.03) (layer "F.Cu") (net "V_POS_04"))
 (segment (start 98.020101 101.697056) (end 98.302944 101.979899) (width 0.03) (layer "F.Cu") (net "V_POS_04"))
 (segment (start 98.302944 101.979899) (end 98.585786 102.262742) (width 0.03) (layer "F.Cu") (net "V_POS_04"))
 (segment (start 98.585786 102.262742) (end 98.868629 102.545584) (width 0.03) (layer "F.Cu") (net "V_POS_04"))
 (segment (start 100.141421 100.424264) (end 100.282843 100.565685) (width 0.03) (layer "F.Cu") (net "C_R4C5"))
 (segment (start 95.615938 95.050253) (end 100.565685 100) (width 0.03) (layer "F.Cu") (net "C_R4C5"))
 (segment (start 93.353196 88.969134) (end 94.060303 89.676241) (width 0.03) (layer "F.Cu") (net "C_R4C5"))
 (segment (start 100.565685 100) (end 100.141421 100.424264) (width 0.03) (layer "F.Cu") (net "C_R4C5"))
 (segment (start 94.060303 89.676241) (end 95.615938 95.050253) (width 0.03) (layer "F.Cu") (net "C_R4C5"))
 (segment (start 95.927065 94.739126) (end 100.311127 99.123188) (width 0.03) (layer "F.Cu") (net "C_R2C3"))
 (segment (start 100.141421 99.292893) (end 100.282843 99.434315) (width 0.03) (layer "F.Cu") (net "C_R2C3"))
 (segment (start 94.625988 89.110556) (end 95.927065 94.739126) (width 0.03) (layer "F.Cu") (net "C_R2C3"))
 (segment (start 93.918882 88.403449) (end 94.625988 89.110556) (width 0.03) (layer "F.Cu") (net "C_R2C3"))
 (segment (start 100.311127 99.123188) (end 100.141421 99.292893) (width 0.03) (layer "F.Cu") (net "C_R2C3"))
 (segment (start 95.757359 103.959798) (end 96.040202 104.242641) (width 0.03) (layer "F.Cu") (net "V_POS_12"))
 (segment (start 96.040202 104.242641) (end 96.323045 104.525483) (width 0.03) (layer "F.Cu") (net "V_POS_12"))
 (segment (start 91.231876 99.434315) (end 95.191674 103.394113) (width 0.03) (layer "F.Cu") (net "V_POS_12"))
 (segment (start 89.251977 94.484567) (end 91.231876 99.434315) (width 0.03) (layer "F.Cu") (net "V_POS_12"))
 (segment (start 95.191674 103.394113) (end 95.474517 103.676955) (width 0.03) (layer "F.Cu") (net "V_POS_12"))
 (segment (start 96.323045 104.525483) (end 96.605887 104.808326) (width 0.03) (layer "F.Cu") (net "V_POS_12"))
 (segment (start 95.474517 103.676955) (end 95.757359 103.959798) (width 0.03) (layer "F.Cu") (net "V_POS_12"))
 (segment (start 88.54487 93.77746) (end 89.251977 94.484567) (width 0.03) (layer "F.Cu") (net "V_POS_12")))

